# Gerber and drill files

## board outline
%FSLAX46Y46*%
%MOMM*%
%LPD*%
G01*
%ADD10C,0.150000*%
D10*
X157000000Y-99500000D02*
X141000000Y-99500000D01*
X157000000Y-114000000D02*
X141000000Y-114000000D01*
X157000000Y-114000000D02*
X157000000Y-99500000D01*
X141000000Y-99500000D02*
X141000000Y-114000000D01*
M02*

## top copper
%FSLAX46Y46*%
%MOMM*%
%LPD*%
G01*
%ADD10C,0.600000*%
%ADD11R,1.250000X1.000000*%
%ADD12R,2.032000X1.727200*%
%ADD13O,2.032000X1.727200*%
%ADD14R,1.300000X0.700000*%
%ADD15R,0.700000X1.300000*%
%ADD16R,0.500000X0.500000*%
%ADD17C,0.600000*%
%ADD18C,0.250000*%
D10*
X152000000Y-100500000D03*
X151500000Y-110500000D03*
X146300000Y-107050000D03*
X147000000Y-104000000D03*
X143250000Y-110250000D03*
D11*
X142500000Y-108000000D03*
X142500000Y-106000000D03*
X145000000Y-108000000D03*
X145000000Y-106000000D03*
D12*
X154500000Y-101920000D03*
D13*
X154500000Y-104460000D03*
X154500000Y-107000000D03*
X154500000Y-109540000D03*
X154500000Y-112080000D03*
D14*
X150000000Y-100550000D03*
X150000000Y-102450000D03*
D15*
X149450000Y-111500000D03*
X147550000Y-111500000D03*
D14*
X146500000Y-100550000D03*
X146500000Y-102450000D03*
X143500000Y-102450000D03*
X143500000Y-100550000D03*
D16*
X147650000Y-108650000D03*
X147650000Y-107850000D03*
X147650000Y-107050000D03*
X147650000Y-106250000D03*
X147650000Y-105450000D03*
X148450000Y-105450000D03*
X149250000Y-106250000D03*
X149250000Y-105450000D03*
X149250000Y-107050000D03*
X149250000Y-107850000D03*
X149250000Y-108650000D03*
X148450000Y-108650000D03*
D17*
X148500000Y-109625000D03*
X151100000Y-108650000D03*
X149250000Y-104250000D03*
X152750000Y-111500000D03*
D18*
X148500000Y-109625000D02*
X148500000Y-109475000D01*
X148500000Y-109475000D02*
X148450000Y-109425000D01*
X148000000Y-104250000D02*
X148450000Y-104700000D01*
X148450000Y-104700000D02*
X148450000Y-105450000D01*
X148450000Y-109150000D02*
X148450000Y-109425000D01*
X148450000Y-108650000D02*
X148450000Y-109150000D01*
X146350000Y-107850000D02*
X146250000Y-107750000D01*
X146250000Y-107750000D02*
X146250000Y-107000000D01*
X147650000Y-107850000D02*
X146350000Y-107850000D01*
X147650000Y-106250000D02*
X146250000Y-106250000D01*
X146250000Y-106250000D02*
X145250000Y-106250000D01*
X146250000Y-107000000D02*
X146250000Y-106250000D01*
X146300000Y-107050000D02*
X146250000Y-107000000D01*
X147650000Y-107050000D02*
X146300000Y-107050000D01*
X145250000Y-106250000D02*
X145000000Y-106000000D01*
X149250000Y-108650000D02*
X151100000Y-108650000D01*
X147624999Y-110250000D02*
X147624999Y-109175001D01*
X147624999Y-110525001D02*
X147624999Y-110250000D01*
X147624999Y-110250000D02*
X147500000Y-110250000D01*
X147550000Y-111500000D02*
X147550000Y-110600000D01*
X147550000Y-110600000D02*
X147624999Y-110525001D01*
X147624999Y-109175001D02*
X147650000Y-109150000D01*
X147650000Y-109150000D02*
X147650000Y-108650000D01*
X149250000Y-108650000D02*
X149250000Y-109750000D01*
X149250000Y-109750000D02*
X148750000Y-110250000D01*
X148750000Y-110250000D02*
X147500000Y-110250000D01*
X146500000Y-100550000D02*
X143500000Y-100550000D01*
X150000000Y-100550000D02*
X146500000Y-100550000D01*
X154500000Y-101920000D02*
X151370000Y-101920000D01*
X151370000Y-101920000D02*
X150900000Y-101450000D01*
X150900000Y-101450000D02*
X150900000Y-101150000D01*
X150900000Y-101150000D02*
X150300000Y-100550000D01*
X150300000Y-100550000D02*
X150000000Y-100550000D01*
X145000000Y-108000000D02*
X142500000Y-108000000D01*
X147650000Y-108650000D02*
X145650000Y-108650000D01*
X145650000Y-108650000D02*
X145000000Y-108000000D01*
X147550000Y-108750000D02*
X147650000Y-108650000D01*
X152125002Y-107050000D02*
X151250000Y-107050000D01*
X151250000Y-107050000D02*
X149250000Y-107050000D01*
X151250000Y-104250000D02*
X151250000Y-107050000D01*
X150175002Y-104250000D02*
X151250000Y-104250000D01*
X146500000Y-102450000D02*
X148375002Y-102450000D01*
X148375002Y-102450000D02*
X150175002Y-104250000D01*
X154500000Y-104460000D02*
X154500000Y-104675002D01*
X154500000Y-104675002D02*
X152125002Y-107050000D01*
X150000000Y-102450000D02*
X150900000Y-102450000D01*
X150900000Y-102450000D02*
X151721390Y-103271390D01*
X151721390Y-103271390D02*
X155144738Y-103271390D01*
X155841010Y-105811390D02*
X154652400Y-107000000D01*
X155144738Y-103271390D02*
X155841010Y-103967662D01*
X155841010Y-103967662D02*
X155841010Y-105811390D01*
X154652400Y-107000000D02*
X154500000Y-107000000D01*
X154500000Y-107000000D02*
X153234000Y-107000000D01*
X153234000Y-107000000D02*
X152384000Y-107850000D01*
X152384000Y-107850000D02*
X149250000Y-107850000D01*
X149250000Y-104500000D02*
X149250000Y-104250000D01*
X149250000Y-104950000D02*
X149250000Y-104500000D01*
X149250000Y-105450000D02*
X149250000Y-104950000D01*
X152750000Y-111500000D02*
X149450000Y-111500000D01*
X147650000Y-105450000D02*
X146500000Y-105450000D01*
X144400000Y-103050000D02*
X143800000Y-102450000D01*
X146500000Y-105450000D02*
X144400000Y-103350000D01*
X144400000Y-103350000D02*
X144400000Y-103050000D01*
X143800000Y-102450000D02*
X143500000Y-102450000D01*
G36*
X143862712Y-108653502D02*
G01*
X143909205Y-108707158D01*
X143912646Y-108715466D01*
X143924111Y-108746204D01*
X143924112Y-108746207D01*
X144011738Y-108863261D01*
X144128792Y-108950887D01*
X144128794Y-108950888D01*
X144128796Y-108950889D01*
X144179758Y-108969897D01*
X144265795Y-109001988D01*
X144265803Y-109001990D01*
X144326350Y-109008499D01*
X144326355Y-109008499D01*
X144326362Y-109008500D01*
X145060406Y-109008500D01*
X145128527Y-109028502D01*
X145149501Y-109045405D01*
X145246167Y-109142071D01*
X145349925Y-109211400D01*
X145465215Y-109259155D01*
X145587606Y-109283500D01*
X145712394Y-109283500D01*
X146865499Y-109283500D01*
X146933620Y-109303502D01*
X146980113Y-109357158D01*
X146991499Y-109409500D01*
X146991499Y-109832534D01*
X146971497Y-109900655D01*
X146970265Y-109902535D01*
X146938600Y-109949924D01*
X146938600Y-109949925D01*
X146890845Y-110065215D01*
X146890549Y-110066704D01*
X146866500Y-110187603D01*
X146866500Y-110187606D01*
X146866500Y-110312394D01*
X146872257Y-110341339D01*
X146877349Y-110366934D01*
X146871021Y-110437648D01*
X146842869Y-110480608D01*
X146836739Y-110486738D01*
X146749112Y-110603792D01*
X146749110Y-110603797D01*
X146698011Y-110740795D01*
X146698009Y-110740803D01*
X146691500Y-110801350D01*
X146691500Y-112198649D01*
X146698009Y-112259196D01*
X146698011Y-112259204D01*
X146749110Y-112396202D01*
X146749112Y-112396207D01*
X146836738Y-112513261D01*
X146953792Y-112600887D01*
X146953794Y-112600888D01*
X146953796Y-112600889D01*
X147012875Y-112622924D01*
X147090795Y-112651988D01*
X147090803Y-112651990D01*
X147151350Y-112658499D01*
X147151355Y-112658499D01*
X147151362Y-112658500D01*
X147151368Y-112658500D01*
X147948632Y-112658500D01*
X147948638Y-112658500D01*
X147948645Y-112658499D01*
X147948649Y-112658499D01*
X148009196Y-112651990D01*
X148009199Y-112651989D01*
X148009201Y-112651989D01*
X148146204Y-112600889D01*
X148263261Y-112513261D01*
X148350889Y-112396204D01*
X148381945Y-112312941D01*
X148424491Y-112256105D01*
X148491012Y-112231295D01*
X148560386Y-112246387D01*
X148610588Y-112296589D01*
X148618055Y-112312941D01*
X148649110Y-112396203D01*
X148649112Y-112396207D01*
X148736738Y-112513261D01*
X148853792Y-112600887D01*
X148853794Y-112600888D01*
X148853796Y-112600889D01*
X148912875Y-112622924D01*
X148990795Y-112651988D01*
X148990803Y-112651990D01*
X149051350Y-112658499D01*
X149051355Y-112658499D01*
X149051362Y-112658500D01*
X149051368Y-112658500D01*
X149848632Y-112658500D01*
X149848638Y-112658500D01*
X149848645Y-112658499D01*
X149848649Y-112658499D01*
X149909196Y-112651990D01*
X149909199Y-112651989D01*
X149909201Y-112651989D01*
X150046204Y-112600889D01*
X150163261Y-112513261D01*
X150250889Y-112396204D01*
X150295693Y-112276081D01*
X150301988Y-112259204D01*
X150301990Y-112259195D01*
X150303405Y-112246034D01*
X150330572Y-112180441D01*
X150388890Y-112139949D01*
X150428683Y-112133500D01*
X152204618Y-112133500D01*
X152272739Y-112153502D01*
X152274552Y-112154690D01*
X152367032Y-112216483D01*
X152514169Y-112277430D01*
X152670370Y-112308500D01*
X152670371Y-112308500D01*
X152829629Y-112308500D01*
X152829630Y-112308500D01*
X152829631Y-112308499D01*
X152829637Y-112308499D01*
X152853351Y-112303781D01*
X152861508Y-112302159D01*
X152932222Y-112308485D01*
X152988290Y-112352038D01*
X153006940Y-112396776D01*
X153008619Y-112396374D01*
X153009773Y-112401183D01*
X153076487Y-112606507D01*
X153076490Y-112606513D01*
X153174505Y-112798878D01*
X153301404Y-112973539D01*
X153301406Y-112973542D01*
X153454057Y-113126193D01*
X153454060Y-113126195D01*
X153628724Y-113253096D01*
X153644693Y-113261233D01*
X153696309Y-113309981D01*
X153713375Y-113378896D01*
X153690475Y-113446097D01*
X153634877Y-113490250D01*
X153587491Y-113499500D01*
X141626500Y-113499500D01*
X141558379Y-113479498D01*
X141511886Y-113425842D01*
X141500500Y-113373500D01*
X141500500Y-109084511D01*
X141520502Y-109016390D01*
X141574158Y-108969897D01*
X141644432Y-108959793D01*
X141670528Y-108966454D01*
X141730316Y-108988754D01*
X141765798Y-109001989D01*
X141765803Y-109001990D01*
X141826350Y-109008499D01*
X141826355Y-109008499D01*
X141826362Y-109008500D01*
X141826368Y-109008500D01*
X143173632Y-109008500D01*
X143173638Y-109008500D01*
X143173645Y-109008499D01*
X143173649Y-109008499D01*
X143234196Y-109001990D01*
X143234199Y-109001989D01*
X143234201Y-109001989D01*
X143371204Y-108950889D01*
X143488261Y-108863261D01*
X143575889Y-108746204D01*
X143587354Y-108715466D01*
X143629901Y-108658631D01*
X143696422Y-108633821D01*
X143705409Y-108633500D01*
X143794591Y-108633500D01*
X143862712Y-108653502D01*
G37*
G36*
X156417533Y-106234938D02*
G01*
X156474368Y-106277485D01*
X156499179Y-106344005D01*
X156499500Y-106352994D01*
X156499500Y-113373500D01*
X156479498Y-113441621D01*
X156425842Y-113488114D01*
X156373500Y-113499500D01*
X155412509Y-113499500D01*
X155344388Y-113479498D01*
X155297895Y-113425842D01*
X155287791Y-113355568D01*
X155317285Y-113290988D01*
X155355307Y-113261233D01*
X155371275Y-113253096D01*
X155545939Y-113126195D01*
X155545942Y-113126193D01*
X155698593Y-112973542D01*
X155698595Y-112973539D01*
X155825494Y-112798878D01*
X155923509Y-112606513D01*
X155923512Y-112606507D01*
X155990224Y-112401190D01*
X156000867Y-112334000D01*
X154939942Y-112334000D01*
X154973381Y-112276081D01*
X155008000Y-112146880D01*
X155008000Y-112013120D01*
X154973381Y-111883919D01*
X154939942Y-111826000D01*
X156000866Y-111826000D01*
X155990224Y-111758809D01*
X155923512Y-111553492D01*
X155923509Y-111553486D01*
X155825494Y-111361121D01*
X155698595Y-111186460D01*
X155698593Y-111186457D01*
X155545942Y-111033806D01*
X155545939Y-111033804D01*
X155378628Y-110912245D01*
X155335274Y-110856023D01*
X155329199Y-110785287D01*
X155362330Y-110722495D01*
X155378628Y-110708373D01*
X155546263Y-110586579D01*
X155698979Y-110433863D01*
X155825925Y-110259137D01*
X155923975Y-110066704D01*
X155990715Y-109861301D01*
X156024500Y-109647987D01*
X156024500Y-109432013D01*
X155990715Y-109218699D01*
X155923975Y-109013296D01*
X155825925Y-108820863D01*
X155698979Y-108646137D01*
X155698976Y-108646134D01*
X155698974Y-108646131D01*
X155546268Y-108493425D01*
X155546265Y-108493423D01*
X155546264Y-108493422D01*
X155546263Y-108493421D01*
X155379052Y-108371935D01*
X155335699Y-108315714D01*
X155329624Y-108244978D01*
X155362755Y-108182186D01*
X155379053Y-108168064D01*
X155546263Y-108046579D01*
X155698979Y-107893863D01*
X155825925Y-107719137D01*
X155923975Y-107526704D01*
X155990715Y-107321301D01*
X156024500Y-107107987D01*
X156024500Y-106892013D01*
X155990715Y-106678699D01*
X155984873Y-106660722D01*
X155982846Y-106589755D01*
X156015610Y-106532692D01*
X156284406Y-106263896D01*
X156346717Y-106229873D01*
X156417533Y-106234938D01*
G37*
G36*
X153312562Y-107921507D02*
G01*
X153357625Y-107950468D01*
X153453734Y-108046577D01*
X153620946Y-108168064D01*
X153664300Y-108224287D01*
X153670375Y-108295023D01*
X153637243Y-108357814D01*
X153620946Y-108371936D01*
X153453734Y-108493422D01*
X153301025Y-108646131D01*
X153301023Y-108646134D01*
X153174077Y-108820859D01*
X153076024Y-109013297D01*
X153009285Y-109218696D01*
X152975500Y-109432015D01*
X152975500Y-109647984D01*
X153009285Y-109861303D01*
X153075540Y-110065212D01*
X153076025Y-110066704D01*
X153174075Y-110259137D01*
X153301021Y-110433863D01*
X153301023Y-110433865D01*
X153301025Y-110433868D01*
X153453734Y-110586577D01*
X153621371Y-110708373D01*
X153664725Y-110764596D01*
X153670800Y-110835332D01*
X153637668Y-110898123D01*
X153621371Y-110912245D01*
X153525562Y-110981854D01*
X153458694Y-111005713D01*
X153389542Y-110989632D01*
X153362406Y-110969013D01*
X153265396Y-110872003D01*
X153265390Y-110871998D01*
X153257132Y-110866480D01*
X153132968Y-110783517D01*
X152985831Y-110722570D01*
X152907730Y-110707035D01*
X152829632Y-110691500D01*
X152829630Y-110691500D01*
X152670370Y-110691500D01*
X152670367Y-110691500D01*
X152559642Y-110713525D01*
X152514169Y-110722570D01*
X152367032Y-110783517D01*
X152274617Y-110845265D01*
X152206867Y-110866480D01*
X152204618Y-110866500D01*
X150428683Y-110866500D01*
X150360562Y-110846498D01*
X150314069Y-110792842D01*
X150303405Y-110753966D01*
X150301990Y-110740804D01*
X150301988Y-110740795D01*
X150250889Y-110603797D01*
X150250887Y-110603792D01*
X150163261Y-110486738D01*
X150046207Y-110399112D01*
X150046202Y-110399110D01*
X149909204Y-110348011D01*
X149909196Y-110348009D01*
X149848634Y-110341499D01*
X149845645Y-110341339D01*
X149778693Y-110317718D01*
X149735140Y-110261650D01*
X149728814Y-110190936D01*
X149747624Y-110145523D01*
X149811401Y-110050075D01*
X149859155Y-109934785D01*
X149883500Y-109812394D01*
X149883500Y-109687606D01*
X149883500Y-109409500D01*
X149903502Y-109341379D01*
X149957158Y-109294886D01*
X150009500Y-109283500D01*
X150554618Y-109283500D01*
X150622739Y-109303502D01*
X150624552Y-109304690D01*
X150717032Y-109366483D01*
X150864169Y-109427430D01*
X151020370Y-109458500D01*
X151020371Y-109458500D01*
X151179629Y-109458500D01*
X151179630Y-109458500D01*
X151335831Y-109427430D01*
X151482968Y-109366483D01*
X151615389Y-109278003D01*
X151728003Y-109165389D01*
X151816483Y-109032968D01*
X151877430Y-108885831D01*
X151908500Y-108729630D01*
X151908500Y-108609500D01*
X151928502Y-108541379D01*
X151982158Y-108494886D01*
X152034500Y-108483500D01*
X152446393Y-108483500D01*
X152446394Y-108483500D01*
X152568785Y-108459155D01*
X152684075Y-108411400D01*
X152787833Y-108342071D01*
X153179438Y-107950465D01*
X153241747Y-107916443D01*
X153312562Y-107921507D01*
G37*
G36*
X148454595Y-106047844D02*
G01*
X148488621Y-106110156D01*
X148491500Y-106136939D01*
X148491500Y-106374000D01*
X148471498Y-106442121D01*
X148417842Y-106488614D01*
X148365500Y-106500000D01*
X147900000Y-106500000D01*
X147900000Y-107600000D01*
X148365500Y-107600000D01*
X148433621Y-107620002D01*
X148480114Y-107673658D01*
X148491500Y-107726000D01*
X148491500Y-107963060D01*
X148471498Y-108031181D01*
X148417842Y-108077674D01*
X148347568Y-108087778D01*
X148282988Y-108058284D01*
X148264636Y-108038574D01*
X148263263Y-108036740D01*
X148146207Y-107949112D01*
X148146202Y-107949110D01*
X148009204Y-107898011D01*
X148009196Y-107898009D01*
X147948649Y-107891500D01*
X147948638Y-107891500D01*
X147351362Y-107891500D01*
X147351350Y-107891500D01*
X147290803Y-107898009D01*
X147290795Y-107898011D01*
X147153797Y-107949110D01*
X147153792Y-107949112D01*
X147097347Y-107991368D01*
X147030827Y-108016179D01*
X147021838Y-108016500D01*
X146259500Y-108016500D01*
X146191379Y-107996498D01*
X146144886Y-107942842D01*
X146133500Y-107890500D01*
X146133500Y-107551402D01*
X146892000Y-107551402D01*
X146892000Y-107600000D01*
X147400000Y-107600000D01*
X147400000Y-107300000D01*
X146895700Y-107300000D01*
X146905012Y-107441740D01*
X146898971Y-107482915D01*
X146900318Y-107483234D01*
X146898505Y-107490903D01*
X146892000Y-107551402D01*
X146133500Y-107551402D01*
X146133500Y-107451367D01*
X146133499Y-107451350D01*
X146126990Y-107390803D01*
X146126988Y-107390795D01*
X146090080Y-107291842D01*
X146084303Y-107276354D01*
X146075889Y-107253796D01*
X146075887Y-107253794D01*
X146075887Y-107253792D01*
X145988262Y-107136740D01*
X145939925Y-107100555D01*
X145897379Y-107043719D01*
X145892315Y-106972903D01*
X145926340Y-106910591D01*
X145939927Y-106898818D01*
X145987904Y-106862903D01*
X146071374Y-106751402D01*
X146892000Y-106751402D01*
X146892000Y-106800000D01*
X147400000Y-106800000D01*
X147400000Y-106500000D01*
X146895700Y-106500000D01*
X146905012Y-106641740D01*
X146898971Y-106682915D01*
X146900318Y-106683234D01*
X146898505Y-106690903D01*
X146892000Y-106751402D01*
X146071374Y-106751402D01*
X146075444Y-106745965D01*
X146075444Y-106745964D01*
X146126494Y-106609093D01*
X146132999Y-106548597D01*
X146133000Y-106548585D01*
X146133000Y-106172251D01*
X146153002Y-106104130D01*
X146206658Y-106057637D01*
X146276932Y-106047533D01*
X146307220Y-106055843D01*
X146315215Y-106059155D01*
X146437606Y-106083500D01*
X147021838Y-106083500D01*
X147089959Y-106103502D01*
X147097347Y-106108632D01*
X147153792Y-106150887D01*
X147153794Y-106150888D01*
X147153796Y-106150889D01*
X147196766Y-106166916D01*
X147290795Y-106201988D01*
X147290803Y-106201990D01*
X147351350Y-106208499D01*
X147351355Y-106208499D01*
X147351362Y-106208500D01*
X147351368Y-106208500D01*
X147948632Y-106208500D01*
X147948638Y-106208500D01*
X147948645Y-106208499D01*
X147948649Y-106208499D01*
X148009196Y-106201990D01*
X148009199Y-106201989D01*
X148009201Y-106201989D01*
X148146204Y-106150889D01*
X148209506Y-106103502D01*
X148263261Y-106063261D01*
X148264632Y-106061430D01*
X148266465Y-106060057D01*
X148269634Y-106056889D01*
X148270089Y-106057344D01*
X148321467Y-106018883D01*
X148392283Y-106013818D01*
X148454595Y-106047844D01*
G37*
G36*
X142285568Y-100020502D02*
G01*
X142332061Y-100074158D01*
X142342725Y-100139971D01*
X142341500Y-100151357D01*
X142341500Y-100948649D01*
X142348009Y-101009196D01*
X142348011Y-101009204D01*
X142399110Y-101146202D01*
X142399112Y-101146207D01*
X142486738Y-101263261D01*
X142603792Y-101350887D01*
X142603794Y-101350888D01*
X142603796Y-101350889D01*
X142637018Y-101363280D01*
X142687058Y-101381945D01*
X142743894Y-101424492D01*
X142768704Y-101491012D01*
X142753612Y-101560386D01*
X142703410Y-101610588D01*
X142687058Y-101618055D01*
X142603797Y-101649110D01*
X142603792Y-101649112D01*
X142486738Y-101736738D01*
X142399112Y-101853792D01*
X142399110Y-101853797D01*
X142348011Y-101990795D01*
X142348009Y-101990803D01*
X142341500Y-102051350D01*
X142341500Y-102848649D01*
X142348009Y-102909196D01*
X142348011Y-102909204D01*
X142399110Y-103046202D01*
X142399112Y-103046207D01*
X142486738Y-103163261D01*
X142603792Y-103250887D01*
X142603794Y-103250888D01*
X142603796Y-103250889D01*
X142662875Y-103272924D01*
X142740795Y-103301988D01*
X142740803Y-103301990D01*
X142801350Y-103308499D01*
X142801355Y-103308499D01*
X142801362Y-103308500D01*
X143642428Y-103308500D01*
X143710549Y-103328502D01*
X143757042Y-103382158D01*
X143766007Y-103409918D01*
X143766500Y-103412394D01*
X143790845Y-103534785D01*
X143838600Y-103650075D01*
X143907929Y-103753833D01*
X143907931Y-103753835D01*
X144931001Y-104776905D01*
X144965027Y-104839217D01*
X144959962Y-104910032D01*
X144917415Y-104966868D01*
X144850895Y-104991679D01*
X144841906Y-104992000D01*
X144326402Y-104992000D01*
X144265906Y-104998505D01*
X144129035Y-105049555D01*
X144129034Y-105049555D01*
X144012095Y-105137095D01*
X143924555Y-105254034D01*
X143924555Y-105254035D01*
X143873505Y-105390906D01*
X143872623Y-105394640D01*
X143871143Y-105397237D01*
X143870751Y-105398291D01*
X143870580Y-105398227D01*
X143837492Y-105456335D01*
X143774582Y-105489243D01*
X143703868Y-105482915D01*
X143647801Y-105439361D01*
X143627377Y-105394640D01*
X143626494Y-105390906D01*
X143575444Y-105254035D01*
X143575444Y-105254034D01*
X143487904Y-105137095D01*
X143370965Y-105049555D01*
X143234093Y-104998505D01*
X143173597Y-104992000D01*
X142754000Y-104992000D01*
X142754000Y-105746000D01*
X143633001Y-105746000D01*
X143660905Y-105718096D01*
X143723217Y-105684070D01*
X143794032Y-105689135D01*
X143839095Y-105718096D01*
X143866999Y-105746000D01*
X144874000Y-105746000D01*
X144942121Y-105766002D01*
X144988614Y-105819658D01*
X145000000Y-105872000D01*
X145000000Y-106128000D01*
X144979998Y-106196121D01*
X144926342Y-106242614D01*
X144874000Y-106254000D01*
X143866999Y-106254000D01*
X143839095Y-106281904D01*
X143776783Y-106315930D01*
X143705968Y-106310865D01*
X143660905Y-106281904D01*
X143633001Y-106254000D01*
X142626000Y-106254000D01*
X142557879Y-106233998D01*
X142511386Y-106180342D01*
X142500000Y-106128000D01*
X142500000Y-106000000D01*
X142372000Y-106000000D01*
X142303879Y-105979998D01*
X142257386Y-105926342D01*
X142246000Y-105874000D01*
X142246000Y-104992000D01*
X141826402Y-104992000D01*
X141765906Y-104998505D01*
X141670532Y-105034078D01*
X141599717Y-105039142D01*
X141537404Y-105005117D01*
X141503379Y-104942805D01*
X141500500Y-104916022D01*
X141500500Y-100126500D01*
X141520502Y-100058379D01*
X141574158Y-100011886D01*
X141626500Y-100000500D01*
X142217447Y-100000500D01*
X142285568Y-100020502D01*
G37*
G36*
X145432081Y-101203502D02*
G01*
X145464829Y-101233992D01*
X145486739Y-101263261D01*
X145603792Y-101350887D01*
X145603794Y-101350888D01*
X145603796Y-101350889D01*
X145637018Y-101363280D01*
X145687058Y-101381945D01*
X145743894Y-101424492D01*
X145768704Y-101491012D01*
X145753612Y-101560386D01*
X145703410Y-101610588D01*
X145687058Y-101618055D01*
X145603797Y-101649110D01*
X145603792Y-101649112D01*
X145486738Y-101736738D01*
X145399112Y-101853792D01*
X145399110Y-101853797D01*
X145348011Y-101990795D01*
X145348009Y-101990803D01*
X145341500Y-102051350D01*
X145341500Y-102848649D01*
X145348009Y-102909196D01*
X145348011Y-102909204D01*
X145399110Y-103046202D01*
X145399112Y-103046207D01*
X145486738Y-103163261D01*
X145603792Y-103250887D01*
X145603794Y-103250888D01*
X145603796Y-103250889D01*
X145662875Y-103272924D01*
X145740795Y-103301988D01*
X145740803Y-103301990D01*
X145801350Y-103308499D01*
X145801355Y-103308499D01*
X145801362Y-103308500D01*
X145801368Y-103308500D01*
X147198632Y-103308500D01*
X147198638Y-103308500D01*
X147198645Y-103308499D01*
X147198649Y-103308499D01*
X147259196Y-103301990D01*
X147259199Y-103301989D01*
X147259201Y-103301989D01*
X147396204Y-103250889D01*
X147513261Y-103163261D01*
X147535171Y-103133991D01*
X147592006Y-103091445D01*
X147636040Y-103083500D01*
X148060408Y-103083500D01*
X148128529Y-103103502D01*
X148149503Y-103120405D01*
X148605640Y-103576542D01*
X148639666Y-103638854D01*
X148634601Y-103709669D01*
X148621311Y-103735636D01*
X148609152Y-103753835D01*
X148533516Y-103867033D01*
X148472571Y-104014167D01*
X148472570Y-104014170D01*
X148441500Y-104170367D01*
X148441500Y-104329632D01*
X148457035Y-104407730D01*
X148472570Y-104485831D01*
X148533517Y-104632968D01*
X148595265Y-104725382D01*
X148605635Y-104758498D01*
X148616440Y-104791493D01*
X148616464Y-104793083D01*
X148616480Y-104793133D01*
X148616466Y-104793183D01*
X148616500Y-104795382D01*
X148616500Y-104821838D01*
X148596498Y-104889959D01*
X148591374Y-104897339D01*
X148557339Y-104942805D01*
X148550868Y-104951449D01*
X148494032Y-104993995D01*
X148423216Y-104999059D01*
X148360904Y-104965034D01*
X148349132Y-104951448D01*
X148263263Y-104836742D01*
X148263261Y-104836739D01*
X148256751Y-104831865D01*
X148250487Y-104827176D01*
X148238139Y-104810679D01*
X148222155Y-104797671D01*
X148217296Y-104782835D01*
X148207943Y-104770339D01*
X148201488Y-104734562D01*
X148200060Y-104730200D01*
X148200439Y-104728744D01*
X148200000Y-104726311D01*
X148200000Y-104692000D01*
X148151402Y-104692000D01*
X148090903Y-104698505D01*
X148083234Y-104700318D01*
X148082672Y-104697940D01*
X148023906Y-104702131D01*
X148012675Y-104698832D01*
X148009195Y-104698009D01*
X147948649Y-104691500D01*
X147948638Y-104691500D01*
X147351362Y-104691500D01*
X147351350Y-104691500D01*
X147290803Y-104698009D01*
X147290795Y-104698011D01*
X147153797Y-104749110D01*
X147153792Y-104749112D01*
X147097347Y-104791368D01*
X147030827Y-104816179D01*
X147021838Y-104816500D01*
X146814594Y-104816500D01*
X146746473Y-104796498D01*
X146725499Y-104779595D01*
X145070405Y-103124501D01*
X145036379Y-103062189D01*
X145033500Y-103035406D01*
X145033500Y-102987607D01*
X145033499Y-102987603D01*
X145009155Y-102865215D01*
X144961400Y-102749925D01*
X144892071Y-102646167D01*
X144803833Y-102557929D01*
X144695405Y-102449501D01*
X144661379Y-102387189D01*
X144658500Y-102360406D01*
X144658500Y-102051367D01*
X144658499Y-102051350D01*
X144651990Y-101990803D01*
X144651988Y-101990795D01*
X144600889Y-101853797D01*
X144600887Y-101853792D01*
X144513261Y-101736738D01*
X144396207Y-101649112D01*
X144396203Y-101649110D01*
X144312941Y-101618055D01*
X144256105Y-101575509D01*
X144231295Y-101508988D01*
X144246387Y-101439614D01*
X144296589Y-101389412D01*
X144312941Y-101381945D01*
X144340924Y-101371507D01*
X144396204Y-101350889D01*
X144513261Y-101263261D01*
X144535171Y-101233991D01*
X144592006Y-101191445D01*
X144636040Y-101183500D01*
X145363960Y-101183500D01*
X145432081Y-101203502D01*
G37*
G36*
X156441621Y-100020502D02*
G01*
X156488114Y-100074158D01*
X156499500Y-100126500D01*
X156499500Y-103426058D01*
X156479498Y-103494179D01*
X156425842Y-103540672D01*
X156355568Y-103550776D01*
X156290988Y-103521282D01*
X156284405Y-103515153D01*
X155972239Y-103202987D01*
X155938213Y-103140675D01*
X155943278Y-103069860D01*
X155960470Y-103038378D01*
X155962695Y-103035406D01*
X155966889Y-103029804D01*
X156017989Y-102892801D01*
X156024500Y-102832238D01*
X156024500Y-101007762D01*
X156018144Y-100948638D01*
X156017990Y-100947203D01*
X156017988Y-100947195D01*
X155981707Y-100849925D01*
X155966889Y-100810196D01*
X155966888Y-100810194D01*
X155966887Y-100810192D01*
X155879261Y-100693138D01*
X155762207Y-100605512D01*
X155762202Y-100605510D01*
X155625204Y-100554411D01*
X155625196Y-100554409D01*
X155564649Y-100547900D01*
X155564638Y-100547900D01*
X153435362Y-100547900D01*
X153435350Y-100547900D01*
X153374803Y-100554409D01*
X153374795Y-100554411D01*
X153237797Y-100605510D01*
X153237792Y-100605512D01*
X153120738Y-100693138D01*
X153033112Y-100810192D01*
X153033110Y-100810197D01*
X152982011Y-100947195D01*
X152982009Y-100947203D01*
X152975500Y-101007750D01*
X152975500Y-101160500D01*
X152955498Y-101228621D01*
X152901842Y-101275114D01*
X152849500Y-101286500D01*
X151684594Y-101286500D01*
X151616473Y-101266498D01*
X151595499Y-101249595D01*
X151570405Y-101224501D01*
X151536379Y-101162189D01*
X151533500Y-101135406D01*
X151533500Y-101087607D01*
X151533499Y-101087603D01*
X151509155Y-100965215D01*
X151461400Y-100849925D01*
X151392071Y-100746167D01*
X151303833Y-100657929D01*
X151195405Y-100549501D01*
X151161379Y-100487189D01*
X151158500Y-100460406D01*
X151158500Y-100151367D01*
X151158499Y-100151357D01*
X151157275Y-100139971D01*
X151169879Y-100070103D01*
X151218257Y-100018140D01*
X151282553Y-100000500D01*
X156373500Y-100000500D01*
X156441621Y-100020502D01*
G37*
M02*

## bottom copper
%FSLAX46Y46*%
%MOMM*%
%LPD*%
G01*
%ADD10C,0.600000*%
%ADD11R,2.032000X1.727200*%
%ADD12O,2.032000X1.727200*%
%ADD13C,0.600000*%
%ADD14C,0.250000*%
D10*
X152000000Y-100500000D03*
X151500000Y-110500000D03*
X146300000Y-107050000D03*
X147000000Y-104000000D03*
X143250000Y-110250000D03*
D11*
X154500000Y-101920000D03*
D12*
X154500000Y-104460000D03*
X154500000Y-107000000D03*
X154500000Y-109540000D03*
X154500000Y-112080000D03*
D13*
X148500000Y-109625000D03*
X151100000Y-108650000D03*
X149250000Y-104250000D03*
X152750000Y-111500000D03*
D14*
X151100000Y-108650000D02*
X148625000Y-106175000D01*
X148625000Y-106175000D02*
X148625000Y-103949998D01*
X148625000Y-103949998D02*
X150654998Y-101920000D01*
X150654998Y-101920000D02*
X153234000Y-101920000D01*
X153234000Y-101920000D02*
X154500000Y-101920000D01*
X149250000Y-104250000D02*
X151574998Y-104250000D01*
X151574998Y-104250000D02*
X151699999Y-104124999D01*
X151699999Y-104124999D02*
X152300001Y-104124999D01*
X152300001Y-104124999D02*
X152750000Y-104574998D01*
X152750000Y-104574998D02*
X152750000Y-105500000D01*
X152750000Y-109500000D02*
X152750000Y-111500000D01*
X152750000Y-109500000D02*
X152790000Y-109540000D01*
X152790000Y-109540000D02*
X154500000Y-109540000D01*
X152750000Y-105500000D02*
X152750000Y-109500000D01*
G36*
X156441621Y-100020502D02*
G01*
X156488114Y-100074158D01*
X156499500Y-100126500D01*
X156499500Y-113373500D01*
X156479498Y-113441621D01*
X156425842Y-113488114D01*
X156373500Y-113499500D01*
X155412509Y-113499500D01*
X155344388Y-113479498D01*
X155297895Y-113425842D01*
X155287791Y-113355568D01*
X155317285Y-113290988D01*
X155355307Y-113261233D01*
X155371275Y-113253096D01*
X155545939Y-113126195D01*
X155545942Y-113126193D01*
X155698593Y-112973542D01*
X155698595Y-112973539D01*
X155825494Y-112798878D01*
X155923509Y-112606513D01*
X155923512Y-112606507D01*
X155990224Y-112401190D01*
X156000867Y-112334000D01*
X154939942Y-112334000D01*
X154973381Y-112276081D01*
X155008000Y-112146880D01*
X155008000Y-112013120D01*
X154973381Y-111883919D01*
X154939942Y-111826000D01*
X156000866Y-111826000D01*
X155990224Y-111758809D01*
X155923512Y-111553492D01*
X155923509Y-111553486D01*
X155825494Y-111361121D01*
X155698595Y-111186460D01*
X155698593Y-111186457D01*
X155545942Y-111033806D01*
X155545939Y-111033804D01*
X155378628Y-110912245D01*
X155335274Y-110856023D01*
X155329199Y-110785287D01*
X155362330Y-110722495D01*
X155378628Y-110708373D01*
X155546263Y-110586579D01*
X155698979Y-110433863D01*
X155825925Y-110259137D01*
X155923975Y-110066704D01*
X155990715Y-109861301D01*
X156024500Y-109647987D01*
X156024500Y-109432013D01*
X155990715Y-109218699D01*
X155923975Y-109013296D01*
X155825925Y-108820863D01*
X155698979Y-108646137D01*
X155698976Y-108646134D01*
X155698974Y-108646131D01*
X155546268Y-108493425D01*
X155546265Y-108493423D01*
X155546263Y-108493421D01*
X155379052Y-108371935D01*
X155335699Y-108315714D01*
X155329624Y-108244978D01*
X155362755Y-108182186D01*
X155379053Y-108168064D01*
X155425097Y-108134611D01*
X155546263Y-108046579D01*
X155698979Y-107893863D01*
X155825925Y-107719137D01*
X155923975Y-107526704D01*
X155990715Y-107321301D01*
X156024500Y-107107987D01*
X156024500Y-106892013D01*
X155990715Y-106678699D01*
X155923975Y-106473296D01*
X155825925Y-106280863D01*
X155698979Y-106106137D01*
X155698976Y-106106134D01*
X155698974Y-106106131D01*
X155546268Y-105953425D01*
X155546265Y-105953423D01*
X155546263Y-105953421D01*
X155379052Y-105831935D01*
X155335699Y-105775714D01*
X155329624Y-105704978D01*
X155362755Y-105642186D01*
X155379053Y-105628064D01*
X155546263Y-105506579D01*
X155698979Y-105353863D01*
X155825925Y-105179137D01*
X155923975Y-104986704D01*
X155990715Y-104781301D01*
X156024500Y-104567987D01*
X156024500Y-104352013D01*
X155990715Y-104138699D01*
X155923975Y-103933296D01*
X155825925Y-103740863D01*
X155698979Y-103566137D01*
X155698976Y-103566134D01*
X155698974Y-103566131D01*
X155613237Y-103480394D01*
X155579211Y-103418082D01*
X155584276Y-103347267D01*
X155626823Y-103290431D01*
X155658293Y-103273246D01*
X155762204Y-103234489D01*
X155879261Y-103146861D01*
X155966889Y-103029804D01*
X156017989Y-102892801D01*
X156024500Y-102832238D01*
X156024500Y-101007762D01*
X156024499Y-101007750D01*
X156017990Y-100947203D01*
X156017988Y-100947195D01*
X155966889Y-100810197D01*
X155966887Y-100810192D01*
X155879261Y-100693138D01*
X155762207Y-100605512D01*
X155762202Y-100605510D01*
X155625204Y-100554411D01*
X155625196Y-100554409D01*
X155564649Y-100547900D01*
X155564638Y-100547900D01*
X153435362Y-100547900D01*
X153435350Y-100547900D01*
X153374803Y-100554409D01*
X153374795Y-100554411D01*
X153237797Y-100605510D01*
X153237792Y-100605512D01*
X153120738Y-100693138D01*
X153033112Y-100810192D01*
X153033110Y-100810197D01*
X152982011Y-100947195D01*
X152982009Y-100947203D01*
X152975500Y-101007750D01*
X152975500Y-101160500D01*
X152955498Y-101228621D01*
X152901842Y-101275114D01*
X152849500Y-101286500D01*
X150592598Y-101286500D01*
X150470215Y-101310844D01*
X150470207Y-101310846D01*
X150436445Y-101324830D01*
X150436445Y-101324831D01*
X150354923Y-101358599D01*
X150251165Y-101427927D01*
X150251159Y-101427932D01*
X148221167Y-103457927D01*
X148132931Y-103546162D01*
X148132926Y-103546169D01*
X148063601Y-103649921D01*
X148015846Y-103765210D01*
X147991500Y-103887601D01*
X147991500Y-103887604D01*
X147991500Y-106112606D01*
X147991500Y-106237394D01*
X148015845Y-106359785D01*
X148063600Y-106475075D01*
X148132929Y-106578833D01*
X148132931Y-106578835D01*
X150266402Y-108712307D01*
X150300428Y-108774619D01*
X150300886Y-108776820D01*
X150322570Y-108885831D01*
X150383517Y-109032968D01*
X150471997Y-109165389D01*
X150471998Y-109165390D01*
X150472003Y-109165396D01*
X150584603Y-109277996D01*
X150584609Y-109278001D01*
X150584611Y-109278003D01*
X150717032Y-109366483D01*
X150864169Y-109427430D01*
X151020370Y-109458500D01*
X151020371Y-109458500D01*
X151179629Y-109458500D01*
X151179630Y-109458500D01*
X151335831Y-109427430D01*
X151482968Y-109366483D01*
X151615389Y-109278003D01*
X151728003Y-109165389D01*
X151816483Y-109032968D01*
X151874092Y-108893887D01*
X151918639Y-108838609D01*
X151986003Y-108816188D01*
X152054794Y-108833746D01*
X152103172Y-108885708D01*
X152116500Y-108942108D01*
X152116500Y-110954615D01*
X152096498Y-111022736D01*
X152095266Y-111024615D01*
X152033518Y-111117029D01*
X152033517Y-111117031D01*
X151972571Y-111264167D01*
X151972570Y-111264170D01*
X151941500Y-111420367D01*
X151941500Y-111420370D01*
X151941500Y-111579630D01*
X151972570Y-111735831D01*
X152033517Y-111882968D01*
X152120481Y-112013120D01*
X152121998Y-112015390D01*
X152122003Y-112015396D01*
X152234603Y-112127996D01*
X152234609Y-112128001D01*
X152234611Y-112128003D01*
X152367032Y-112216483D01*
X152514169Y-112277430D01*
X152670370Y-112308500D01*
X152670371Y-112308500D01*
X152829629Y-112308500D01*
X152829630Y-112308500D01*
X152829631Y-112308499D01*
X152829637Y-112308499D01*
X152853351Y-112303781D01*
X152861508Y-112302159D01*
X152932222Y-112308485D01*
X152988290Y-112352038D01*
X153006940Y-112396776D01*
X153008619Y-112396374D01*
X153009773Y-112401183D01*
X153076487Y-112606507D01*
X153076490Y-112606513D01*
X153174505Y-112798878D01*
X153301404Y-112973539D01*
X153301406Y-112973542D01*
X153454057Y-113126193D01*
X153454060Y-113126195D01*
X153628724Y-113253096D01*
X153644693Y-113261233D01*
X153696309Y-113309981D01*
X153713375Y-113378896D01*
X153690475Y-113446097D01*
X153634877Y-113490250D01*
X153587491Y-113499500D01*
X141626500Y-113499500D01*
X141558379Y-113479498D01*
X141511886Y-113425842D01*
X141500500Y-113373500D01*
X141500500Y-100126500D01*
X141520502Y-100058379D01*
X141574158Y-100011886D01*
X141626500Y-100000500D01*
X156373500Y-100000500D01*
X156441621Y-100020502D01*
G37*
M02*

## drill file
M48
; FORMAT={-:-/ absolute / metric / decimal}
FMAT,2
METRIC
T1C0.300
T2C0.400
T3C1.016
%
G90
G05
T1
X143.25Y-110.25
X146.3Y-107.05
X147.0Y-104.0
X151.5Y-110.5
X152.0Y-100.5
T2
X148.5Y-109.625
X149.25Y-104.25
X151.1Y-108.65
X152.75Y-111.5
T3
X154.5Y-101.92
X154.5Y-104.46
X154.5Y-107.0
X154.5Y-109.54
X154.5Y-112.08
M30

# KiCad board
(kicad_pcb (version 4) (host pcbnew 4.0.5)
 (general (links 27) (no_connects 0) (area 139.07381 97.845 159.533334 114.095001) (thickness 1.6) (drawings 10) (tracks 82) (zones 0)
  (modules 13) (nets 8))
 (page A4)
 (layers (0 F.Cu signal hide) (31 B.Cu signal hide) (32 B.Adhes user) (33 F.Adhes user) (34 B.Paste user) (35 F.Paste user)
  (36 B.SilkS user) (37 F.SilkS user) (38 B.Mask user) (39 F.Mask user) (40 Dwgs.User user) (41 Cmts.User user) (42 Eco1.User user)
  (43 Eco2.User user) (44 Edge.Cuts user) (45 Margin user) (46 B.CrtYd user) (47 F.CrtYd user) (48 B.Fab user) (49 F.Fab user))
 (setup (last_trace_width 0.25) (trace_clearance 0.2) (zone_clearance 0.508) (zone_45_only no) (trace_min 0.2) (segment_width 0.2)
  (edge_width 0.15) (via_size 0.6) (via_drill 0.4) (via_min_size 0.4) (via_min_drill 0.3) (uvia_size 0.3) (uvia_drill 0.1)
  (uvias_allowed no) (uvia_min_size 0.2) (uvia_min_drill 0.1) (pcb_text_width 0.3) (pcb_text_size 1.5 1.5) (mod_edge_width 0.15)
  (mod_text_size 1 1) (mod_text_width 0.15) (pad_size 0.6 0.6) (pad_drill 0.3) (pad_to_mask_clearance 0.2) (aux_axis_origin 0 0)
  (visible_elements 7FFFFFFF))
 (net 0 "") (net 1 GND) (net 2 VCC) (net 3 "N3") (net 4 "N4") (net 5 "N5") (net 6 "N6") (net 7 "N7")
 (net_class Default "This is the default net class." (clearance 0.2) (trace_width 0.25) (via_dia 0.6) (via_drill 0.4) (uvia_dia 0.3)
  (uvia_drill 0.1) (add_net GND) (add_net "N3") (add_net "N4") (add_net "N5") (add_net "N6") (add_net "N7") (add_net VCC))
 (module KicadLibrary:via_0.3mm (layer F.Cu) (at 152 100.5)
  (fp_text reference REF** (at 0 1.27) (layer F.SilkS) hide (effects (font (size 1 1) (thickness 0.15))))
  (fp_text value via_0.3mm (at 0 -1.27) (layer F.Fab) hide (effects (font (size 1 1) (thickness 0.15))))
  (pad 1 thru_hole circle (at 0 0) (size 0.6 0.6) (drill 0.3) (layers *.Cu) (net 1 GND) (zone_connect 2)))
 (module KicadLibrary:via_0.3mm (layer F.Cu) (at 151.5 110.5)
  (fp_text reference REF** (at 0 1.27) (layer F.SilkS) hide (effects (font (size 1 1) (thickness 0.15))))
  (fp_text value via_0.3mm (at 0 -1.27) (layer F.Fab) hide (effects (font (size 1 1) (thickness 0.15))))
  (pad 1 thru_hole circle (at 0 0) (size 0.6 0.6) (drill 0.3) (layers *.Cu) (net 1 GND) (zone_connect 2)))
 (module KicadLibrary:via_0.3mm (layer F.Cu) (at 146.3 107.05)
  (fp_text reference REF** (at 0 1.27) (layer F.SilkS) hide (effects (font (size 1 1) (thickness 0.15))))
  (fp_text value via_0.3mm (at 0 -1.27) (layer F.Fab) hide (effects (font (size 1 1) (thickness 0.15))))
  (pad 1 thru_hole circle (at 0 0) (size 0.6 0.6) (drill 0.3) (layers *.Cu) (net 1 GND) (zone_connect 2)))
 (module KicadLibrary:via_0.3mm (layer F.Cu) (at 147 104)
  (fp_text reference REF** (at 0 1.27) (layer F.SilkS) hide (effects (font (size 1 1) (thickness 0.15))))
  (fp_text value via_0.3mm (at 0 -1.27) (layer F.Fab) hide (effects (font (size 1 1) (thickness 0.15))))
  (pad 1 thru_hole circle (at 0 0) (size 0.6 0.6) (drill 0.3) (layers *.Cu) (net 1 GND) (zone_connect 2)))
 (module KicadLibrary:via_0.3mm (layer F.Cu) (at 143.25 110.25)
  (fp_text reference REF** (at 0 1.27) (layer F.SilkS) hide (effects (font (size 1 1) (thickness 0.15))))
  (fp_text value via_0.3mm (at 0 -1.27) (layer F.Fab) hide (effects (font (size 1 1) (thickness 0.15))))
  (pad 1 thru_hole circle (at 0 0) (size 0.6 0.6) (drill 0.3) (layers *.Cu) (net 1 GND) (zone_connect 2)))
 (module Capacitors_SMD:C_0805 (layer F.Cu) (at 142.5 107 90)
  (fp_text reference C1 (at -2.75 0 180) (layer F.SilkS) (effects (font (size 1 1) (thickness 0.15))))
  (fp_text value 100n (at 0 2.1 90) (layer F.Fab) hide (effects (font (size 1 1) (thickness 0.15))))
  (pad 1 smd rect (at -1 0 90) (size 1 1.25) (layers F.Cu F.Paste F.Mask) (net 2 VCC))
  (pad 2 smd rect (at 1 0 90) (size 1 1.25) (layers F.Cu F.Paste F.Mask) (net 1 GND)))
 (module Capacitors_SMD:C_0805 (layer F.Cu) (at 145 107 90)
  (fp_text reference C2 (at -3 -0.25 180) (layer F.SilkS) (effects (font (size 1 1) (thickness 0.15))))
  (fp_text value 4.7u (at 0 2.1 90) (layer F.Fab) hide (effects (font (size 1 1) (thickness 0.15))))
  (pad 1 smd rect (at -1 0 90) (size 1 1.25) (layers F.Cu F.Paste F.Mask) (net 2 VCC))
  (pad 2 smd rect (at 1 0 90) (size 1 1.25) (layers F.Cu F.Paste F.Mask) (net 1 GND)))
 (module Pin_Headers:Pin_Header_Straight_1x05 (layer F.Cu) (at 154.5 101.92)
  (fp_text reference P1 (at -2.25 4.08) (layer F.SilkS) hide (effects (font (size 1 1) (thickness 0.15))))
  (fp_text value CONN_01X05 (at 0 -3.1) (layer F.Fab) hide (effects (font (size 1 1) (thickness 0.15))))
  (pad 1 thru_hole rect (at 0 0) (size 2.032 1.7272) (drill 1.016) (layers *.Cu *.Mask) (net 2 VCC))
  (pad 2 thru_hole oval (at 0 2.54) (size 2.032 1.7272) (drill 1.016) (layers *.Cu *.Mask) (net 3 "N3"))
  (pad 3 thru_hole oval (at 0 5.08) (size 2.032 1.7272) (drill 1.016) (layers *.Cu *.Mask) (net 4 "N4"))
  (pad 4 thru_hole oval (at 0 7.62) (size 2.032 1.7272) (drill 1.016) (layers *.Cu *.Mask) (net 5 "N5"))
  (pad 5 thru_hole oval (at 0 10.16) (size 2.032 1.7272) (drill 1.016) (layers *.Cu *.Mask) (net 1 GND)))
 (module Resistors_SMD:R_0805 (layer F.Cu) (at 150 101.5 270)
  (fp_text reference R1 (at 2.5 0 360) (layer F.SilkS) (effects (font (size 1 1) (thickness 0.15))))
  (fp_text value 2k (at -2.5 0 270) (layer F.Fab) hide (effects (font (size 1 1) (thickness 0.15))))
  (pad 1 smd rect (at -0.95 0 270) (size 0.7 1.3) (layers F.Cu F.Paste F.Mask) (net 2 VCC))
  (pad 2 smd rect (at 0.95 0 270) (size 0.7 1.3) (layers F.Cu F.Paste F.Mask) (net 4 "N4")))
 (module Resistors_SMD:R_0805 (layer F.Cu) (at 148.5 111.5 180)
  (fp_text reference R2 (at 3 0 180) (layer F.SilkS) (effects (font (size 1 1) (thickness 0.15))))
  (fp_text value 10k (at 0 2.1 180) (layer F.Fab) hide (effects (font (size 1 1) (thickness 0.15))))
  (pad 1 smd rect (at -0.95 0 180) (size 0.7 1.3) (layers F.Cu F.Paste F.Mask) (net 5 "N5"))
  (pad 2 smd rect (at 0.95 0 180) (size 0.7 1.3) (layers F.Cu F.Paste F.Mask) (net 2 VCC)))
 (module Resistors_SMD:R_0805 (layer F.Cu) (at 146.5 101.5 270)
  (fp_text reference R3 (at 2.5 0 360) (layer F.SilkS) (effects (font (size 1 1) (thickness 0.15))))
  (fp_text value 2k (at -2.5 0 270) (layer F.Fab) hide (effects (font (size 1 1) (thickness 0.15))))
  (pad 1 smd rect (at -0.95 0 270) (size 0.7 1.3) (layers F.Cu F.Paste F.Mask) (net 2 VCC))
  (pad 2 smd rect (at 0.95 0 270) (size 0.7 1.3) (layers F.Cu F.Paste F.Mask) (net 3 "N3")))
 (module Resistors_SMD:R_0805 (layer F.Cu) (at 143.5 101.5 90)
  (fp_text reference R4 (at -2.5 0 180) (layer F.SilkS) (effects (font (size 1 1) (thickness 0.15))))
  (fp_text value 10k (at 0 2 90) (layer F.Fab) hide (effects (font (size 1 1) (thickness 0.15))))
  (pad 1 smd rect (at -0.95 0 90) (size 0.7 1.3) (layers F.Cu F.Paste F.Mask) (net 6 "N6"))
  (pad 2 smd rect (at 0.95 0 90) (size 0.7 1.3) (layers F.Cu F.Paste F.Mask) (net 2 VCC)))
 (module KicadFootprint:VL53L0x (layer F.Cu) (at 148.5 107 90)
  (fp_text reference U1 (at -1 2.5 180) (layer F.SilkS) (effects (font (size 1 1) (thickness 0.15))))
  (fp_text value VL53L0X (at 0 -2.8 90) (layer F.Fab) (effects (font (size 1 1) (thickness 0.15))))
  (pad 1 smd rect (at -1.65 -0.85 90) (size 0.5 0.5) (layers F.Cu F.Paste F.Mask) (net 2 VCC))
  (pad 2 smd rect (at -0.85 -0.85 90) (size 0.5 0.5) (layers F.Cu F.Paste F.Mask) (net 1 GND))
  (pad 3 smd rect (at -0.05 -0.85 90) (size 0.5 0.5) (layers F.Cu F.Paste F.Mask) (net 1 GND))
  (pad 4 smd rect (at 0.75 -0.85 90) (size 0.5 0.5) (layers F.Cu F.Paste F.Mask) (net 1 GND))
  (pad 5 smd rect (at 1.55 -0.85 90) (size 0.5 0.5) (layers F.Cu F.Paste F.Mask) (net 6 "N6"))
  (pad 6 smd rect (at 1.55 -0.05 90) (size 0.5 0.5) (layers F.Cu F.Paste F.Mask) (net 1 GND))
  (pad 8 smd rect (at 0.75 0.75 90) (size 0.5 0.5) (layers F.Cu F.Paste F.Mask) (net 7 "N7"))
  (pad 7 smd rect (at 1.55 0.75 90) (size 0.5 0.5) (layers F.Cu F.Paste F.Mask) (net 5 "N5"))
  (pad 9 smd rect (at -0.05 0.75 90) (size 0.5 0.5) (layers F.Cu F.Paste F.Mask) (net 3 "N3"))
  (pad 10 smd rect (at -0.85 0.75 90) (size 0.5 0.5) (layers F.Cu F.Paste F.Mask) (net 4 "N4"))
  (pad 11 smd rect (at -1.65 0.75 90) (size 0.5 0.5) (layers F.Cu F.Paste F.Mask) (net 2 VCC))
  (pad 12 smd rect (at -1.65 -0.05 90) (size 0.5 0.5) (layers F.Cu F.Paste F.Mask) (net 1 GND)))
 (gr_line (start 157 99.5) (end 141 99.5) (layer Edge.Cuts) (width 0.15))
 (gr_line (start 157 114) (end 141 114) (layer Edge.Cuts) (width 0.15))
 (gr_line (start 157 114) (end 157 99.5) (layer Edge.Cuts) (width 0.15))
 (gr_line (start 141 99.5) (end 141 114) (layer Edge.Cuts) (width 0.15))
 (segment (start 148.5 109.625) (end 148.5 109.475) (width 0.25) (layer F.Cu) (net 1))
 (segment (start 148.5 109.475) (end 148.45 109.425) (width 0.25) (layer F.Cu) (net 1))
 (segment (start 148 104.25) (end 148.45 104.7) (width 0.25) (layer F.Cu) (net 1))
 (segment (start 148.45 104.7) (end 148.45 105.45) (width 0.25) (layer F.Cu) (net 1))
 (segment (start 148.45 109.15) (end 148.45 109.425) (width 0.25) (layer F.Cu) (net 1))
 (via (at 148.5 109.625) (size 0.6) (drill 0.4) (layers F.Cu B.Cu) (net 1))
 (segment (start 148.45 108.65) (end 148.45 109.15) (width 0.25) (layer F.Cu) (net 1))
 (segment (start 146.35 107.85) (end 146.25 107.75) (width 0.25) (layer F.Cu) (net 1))
 (segment (start 146.25 107.75) (end 146.25 107) (width 0.25) (layer F.Cu) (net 1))
 (segment (start 147.65 107.85) (end 146.35 107.85) (width 0.25) (layer F.Cu) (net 1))
 (segment (start 147.65 106.25) (end 146.25 106.25) (width 0.25) (layer F.Cu) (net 1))
 (segment (start 146.25 106.25) (end 145.25 106.25) (width 0.25) (layer F.Cu) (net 1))
 (segment (start 146.25 107) (end 146.25 106.25) (width 0.25) (layer F.Cu) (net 1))
 (segment (start 146.3 107.05) (end 146.25 107) (width 0.25) (layer F.Cu) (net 1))
 (segment (start 147.65 107.05) (end 146.3 107.05) (width 0.25) (layer F.Cu) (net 1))
 (segment (start 145.25 106.25) (end 145 106) (width 0.25) (layer F.Cu) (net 1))
 (segment (start 151.1 108.65) (end 148.625 106.175) (width 0.25) (layer B.Cu) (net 2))
 (segment (start 148.625 106.175) (end 148.625 103.949998) (width 0.25) (layer B.Cu) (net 2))
 (segment (start 148.625 103.949998) (end 150.654998 101.92) (width 0.25) (layer B.Cu) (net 2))
 (segment (start 150.654998 101.92) (end 153.234 101.92) (width 0.25) (layer B.Cu) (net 2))
 (segment (start 153.234 101.92) (end 154.5 101.92) (width 0.25) (layer B.Cu) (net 2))
 (via (at 151.1 108.65) (size 0.6) (drill 0.4) (layers F.Cu B.Cu) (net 2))
 (segment (start 149.25 108.65) (end 151.1 108.65) (width 0.25) (layer F.Cu) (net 2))
 (segment (start 147.624999 110.25) (end 147.624999 109.175001) (width 0.25) (layer F.Cu) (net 2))
 (segment (start 147.624999 110.525001) (end 147.624999 110.25) (width 0.25) (layer F.Cu) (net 2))
 (segment (start 147.624999 110.25) (end 147.5 110.25) (width 0.25) (layer F.Cu) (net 2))
 (segment (start 147.55 111.5) (end 147.55 110.6) (width 0.25) (layer F.Cu) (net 2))
 (segment (start 147.55 110.6) (end 147.624999 110.525001) (width 0.25) (layer F.Cu) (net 2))
 (segment (start 147.624999 109.175001) (end 147.65 109.15) (width 0.25) (layer F.Cu) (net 2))
 (segment (start 147.65 109.15) (end 147.65 108.65) (width 0.25) (layer F.Cu) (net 2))
 (segment (start 149.25 108.65) (end 149.25 109.75) (width 0.25) (layer F.Cu) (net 2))
 (segment (start 149.25 109.75) (end 148.75 110.25) (width 0.25) (layer F.Cu) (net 2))
 (segment (start 148.75 110.25) (end 147.5 110.25) (width 0.25) (layer F.Cu) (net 2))
 (segment (start 146.5 100.55) (end 143.5 100.55) (width 0.25) (layer F.Cu) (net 2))
 (segment (start 150 100.55) (end 146.5 100.55) (width 0.25) (layer F.Cu) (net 2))
 (segment (start 154.5 101.92) (end 151.37 101.92) (width 0.25) (layer F.Cu) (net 2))
 (segment (start 151.37 101.92) (end 150.9 101.45) (width 0.25) (layer F.Cu) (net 2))
 (segment (start 150.9 101.45) (end 150.9 101.15) (width 0.25) (layer F.Cu) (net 2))
 (segment (start 150.9 101.15) (end 150.3 100.55) (width 0.25) (layer F.Cu) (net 2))
 (segment (start 150.3 100.55) (end 150 100.55) (width 0.25) (layer F.Cu) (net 2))
 (segment (start 145 108) (end 142.5 108) (width 0.25) (layer F.Cu) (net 2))
 (segment (start 147.65 108.65) (end 145.65 108.65) (width 0.25) (layer F.Cu) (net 2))
 (segment (start 145.65 108.65) (end 145 108) (width 0.25) (layer F.Cu) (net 2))
 (segment (start 147.55 108.75) (end 147.65 108.65) (width 0.25) (layer F.Cu) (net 2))
 (segment (start 152.125002 107.05) (end 151.25 107.05) (width 0.25) (layer F.Cu) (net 3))
 (segment (start 151.25 107.05) (end 149.25 107.05) (width 0.25) (layer F.Cu) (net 3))
 (segment (start 151.25 104.25) (end 151.25 107.05) (width 0.25) (layer F.Cu) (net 3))
 (segment (start 150.175002 104.25) (end 151.25 104.25) (width 0.25) (layer F.Cu) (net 3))
 (segment (start 146.5 102.45) (end 148.375002 102.45) (width 0.25) (layer F.Cu) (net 3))
 (segment (start 148.375002 102.45) (end 150.175002 104.25) (width 0.25) (layer F.Cu) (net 3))
 (segment (start 154.5 104.46) (end 154.5 104.675002) (width 0.25) (layer F.Cu) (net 3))
 (segment (start 154.5 104.675002) (end 152.125002 107.05) (width 0.25) (layer F.Cu) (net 3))
 (segment (start 150 102.45) (end 150.9 102.45) (width 0.25) (layer F.Cu) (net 4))
 (segment (start 150.9 102.45) (end 151.72139 103.27139) (width 0.25) (layer F.Cu) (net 4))
 (segment (start 151.72139 103.27139) (end 155.144738 103.27139) (width 0.25) (layer F.Cu) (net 4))
 (segment (start 155.84101 105.81139) (end 154.6524 107) (width 0.25) (layer F.Cu) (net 4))
 (segment (start 155.144738 103.27139) (end 155.84101 103.967662) (width 0.25) (layer F.Cu) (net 4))
 (segment (start 155.84101 103.967662) (end 155.84101 105.81139) (width 0.25) (layer F.Cu) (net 4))
 (segment (start 154.6524 107) (end 154.5 107) (width 0.25) (layer F.Cu) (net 4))
 (segment (start 154.5 107) (end 153.234 107) (width 0.25) (layer F.Cu) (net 4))
 (segment (start 153.234 107) (end 152.384 107.85) (width 0.25) (layer F.Cu) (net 4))
 (segment (start 152.384 107.85) (end 149.25 107.85) (width 0.25) (layer F.Cu) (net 4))
 (segment (start 149.25 104.25) (end 151.574998 104.25) (width 0.25) (layer B.Cu) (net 5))
 (segment (start 151.574998 104.25) (end 151.699999 104.124999) (width 0.25) (layer B.Cu) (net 5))
 (segment (start 151.699999 104.124999) (end 152.300001 104.124999) (width 0.25) (layer B.Cu) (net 5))
 (segment (start 152.300001 104.124999) (end 152.75 104.574998) (width 0.25) (layer B.Cu) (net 5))
 (segment (start 152.75 104.574998) (end 152.75 105.5) (width 0.25) (layer B.Cu) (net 5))
 (segment (start 149.25 104.5) (end 149.25 104.25) (width 0.25) (layer F.Cu) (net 5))
 (via (at 149.25 104.25) (size 0.6) (drill 0.4) (layers F.Cu B.Cu) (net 5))
 (segment (start 149.25 104.95) (end 149.25 104.5) (width 0.25) (layer F.Cu) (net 5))
 (segment (start 149.25 105.45) (end 149.25 104.95) (width 0.25) (layer F.Cu) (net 5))
 (segment (start 152.75 111.5) (end 149.45 111.5) (width 0.25) (layer F.Cu) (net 5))
 (via (at 152.75 111.5) (size 0.6) (drill 0.4) (layers F.Cu B.Cu) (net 5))
 (segment (start 152.75 109.5) (end 152.75 111.5) (width 0.25) (layer B.Cu) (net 5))
 (segment (start 152.75 109.5) (end 152.79 109.54) (width 0.25) (layer B.Cu) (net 5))
 (segment (start 152.79 109.54) (end 154.5 109.54) (width 0.25) (layer B.Cu) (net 5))
 (segment (start 152.75 105.5) (end 152.75 109.5) (width 0.25) (layer B.Cu) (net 5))
 (segment (start 147.65 105.45) (end 146.5 105.45) (width 0.25) (layer F.Cu) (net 6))
 (segment (start 144.4 103.05) (end 143.8 102.45) (width 0.25) (layer F.Cu) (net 6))
 (segment (start 146.5 105.45) (end 144.4 103.35) (width 0.25) (layer F.Cu) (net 6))
 (segment (start 144.4 103.35) (end 144.4 103.05) (width 0.25) (layer F.Cu) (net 6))
 (segment (start 143.8 102.45) (end 143.5 102.45) (width 0.25) (layer F.Cu) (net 6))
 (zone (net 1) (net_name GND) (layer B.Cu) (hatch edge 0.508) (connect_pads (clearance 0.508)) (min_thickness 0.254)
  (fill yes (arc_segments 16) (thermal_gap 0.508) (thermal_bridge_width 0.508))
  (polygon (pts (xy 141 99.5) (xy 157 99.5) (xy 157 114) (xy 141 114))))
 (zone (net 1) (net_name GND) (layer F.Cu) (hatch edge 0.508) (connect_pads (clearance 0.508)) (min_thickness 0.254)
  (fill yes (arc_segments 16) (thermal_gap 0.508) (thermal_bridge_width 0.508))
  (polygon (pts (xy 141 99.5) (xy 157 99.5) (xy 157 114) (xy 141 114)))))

